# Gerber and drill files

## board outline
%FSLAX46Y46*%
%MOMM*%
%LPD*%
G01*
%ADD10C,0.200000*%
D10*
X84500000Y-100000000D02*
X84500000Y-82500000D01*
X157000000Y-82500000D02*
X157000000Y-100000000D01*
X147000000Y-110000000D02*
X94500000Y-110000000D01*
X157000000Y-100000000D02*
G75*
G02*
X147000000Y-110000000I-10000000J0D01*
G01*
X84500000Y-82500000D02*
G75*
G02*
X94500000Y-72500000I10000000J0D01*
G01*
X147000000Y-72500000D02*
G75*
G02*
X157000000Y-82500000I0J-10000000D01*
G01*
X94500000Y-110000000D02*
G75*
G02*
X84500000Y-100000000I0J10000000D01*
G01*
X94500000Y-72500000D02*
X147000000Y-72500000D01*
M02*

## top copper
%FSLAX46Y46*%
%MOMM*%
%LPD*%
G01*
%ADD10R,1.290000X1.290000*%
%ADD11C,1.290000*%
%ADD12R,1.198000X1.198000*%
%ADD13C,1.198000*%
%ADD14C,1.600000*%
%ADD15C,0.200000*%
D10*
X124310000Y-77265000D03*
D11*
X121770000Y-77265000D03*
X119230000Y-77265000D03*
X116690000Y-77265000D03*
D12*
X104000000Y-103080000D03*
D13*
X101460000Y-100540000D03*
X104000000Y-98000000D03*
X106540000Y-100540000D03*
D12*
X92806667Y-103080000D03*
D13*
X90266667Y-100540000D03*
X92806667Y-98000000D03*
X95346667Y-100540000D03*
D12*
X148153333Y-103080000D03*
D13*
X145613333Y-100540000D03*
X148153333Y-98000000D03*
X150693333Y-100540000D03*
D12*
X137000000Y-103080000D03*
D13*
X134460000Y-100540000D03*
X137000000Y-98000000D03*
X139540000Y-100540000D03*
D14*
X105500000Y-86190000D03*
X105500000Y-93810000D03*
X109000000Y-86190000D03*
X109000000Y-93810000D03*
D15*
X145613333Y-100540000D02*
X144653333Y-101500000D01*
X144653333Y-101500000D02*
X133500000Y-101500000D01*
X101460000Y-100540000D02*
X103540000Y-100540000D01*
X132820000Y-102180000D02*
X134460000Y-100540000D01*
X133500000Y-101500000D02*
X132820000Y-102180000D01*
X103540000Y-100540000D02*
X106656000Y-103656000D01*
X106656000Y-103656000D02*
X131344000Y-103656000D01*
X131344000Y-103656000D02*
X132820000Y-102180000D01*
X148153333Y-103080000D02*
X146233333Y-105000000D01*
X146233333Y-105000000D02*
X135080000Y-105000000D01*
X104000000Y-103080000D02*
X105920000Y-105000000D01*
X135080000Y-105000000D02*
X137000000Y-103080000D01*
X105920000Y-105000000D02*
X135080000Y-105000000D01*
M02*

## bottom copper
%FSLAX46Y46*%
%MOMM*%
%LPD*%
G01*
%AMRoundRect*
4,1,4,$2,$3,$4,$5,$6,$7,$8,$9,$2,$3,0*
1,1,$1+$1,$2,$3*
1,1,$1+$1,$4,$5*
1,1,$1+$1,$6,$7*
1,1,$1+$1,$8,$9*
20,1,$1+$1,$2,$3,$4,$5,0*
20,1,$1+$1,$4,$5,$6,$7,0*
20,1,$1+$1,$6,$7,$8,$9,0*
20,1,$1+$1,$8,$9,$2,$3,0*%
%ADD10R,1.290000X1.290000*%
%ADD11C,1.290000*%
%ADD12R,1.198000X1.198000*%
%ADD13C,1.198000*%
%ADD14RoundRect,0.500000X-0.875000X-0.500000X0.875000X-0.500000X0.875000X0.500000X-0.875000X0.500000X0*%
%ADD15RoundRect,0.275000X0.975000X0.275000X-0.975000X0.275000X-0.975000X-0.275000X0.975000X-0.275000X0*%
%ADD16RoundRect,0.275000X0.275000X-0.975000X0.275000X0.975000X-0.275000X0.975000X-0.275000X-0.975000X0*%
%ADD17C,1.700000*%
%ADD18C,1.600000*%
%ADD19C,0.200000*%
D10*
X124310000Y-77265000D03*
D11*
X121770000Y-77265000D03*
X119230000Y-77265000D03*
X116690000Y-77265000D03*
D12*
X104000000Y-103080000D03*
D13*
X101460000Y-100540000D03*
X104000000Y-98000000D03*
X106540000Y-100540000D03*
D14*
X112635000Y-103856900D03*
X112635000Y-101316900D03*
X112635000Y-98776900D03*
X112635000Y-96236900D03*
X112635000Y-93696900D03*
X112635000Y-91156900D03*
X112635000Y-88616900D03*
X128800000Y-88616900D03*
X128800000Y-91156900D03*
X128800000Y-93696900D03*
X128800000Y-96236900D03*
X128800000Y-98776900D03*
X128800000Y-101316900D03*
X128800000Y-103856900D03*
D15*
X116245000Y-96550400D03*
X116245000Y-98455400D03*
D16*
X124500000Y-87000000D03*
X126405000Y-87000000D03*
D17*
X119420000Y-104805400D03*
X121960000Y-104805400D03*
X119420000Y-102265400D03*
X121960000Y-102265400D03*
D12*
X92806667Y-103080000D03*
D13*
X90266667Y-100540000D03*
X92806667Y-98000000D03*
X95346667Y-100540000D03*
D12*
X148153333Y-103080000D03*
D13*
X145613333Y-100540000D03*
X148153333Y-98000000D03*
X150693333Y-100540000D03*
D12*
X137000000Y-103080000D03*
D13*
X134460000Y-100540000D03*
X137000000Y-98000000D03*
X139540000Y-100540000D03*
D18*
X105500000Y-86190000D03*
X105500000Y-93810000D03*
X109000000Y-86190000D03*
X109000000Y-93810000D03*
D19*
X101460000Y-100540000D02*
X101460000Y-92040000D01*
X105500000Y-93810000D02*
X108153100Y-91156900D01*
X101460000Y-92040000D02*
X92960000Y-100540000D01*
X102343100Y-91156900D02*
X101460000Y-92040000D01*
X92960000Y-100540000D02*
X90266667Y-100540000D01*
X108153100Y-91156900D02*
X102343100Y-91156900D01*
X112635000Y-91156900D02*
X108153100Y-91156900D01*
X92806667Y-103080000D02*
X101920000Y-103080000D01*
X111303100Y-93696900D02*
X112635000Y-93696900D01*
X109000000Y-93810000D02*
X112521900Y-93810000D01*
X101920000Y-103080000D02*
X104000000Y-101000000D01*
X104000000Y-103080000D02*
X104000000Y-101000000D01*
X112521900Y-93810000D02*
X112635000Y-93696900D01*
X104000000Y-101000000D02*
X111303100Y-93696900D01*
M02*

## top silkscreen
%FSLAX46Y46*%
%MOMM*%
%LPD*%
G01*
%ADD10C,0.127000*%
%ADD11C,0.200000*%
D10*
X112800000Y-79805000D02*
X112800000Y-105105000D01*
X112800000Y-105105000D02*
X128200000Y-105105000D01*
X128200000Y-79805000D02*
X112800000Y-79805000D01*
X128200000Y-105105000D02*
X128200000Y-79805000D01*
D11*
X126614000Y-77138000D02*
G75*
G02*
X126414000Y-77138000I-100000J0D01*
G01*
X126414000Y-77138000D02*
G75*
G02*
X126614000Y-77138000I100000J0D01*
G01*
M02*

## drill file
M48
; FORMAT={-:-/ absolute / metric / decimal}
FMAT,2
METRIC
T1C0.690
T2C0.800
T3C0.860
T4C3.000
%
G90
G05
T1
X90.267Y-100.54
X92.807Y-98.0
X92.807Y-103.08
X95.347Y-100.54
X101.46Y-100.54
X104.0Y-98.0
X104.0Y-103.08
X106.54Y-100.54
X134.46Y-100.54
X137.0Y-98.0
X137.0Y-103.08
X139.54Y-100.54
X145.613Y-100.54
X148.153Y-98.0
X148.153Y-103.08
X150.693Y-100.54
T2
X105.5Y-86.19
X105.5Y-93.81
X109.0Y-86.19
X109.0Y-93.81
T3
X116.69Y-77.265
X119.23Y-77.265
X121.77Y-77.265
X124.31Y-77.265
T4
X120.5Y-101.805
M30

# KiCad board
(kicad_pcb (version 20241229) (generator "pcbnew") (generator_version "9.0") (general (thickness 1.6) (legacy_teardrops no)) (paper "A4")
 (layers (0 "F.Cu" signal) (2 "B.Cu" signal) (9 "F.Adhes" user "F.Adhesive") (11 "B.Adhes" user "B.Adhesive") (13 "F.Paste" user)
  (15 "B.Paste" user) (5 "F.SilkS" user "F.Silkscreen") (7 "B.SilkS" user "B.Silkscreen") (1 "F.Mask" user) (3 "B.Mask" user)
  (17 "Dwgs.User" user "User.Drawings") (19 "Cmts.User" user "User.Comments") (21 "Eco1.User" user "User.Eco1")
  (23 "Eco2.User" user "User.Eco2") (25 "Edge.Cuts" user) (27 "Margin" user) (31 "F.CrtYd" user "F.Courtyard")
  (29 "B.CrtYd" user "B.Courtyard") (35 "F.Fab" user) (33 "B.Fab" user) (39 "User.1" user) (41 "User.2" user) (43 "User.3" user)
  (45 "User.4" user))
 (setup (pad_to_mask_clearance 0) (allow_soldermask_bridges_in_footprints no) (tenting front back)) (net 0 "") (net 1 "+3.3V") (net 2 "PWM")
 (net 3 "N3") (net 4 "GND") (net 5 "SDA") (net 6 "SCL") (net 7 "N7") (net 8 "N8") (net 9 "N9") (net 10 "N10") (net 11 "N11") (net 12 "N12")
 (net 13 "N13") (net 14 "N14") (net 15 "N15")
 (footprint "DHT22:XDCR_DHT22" (layer "F.Cu") (at 120.5 92.455 180)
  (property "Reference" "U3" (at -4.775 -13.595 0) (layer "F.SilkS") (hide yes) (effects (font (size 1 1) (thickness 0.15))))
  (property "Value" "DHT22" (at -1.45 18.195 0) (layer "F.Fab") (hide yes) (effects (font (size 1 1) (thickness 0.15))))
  (fp_line (start 7.7 12.65) (end 7.7 -12.65) (stroke (width 0.127) (type solid)) (layer "F.SilkS"))
  (fp_line (start 7.7 -12.65) (end -7.7 -12.65) (stroke (width 0.127) (type solid)) (layer "F.SilkS"))
  (fp_line (start -7.7 12.65) (end 7.7 12.65) (stroke (width 0.127) (type solid)) (layer "F.SilkS"))
  (fp_line (start -7.7 -12.65) (end -7.7 12.65) (stroke (width 0.127) (type solid)) (layer "F.SilkS"))
  (fp_circle (center -6.014 15.317) (end -5.914 15.317) (stroke (width 0.2) (type solid)) (fill no) (layer "F.SilkS"))
  (pad "" np_thru_hole circle (at 0 -9.35 180) (size 3 3) (drill 3) (layers "*.Cu" "*.Mask"))
  (pad "1" thru_hole rect (at -3.81 15.19 180) (size 1.29 1.29) (drill 0.86) (layers "*.Cu" "*.Mask") (remove_unused_layers no)
   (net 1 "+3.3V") (solder_mask_margin 0.102))
  (pad "2" thru_hole circle (at -1.27 15.19 180) (size 1.29 1.29) (drill 0.86) (layers "*.Cu" "*.Mask") (remove_unused_layers no)
   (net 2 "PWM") (solder_mask_margin 0.102))
  (pad "3" thru_hole circle (at 1.27 15.19 180) (size 1.29 1.29) (drill 0.86) (layers "*.Cu" "*.Mask") (remove_unused_layers no)
   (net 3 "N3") (solder_mask_margin 0.102))
  (pad "4" thru_hole circle (at 3.81 15.19 180) (size 1.29 1.29) (drill 0.86) (layers "*.Cu" "*.Mask") (remove_unused_layers no)
   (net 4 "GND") (solder_mask_margin 0.102)))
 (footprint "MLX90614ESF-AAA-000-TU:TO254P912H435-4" (layer "B.Cu") (at 104 100.54 90)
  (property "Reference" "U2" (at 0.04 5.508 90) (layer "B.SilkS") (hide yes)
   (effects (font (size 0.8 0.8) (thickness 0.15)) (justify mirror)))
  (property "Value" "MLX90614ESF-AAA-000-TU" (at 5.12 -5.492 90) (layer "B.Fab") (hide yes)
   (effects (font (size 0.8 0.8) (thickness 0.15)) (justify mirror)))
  (pad "1" thru_hole rect (at -2.54 0 90) (size 1.198 1.198) (drill 0.69) (layers "*.Cu" "*.Mask") (remove_unused_layers no) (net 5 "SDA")
   (solder_mask_margin 0.102))
  (pad "2" thru_hole circle (at 0 -2.54 90) (size 1.198 1.198) (drill 0.69) (layers "*.Cu" "*.Mask") (remove_unused_layers no) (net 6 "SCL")
   (solder_mask_margin 0.102))
  (pad "3" thru_hole circle (at 2.54 0 90) (size 1.198 1.198) (drill 0.69) (layers "*.Cu" "*.Mask") (remove_unused_layers no)
   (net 1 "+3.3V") (solder_mask_margin 0.102))
  (pad "4" thru_hole circle (at 0 2.54 90) (size 1.198 1.198) (drill 0.69) (layers "*.Cu" "*.Mask") (remove_unused_layers no) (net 4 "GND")
   (solder_mask_margin 0.102)))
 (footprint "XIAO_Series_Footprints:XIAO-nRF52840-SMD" (layer "B.Cu") (at 111.8 85.7369)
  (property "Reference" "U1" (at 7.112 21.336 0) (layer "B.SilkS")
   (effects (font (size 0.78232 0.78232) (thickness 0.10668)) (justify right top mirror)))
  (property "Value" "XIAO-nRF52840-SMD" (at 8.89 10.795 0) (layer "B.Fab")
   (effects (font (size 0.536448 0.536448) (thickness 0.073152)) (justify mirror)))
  (pad "1" smd roundrect (at 0.835 18.12) (size 2.75 2) (layers "B.Cu" "B.Mask" "B.Paste") (roundrect_rratio 0.25) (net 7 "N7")
   (solder_mask_margin 0.0508) (thermal_bridge_angle 45))
  (pad "2" smd roundrect (at 0.835 15.58) (size 2.75 2) (layers "B.Cu" "B.Mask" "B.Paste") (roundrect_rratio 0.25) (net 2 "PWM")
   (solder_mask_margin 0.0508) (thermal_bridge_angle 45))
  (pad "3" smd roundrect (at 0.835 13.04) (size 2.75 2) (layers "B.Cu" "B.Mask" "B.Paste") (roundrect_rratio 0.25) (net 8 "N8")
   (solder_mask_margin 0.0508) (thermal_bridge_angle 45))
  (pad "4" smd roundrect (at 0.835 10.5) (size 2.75 2) (layers "B.Cu" "B.Mask" "B.Paste") (roundrect_rratio 0.25) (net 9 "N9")
   (solder_mask_margin 0.0508) (thermal_bridge_angle 45))
  (pad "5" smd roundrect (at 0.835 7.96) (size 2.75 2) (layers "B.Cu" "B.Mask" "B.Paste") (roundrect_rratio 0.25) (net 5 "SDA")
   (solder_mask_margin 0.0508) (thermal_bridge_angle 45))
  (pad "6" smd roundrect (at 0.835 5.42) (size 2.75 2) (layers "B.Cu" "B.Mask" "B.Paste") (roundrect_rratio 0.25) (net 6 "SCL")
   (solder_mask_margin 0.0508) (thermal_bridge_angle 45))
  (pad "7" smd roundrect (at 0.835 2.88) (size 2.75 2) (layers "B.Cu" "B.Mask" "B.Paste") (roundrect_rratio 0.25) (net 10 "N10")
   (solder_mask_margin 0.0508) (thermal_bridge_angle 45))
  (pad "8" smd roundrect (at 17 2.88) (size 2.75 2) (layers "B.Cu" "B.Mask" "B.Paste") (roundrect_rratio 0.25) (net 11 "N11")
   (solder_mask_margin 0.0508) (thermal_bridge_angle 45))
  (pad "9" smd roundrect (at 17 5.42) (size 2.75 2) (layers "B.Cu" "B.Mask" "B.Paste") (roundrect_rratio 0.25) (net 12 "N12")
   (solder_mask_margin 0.0508) (thermal_bridge_angle 45))
  (pad "10" smd roundrect (at 17 7.96) (size 2.75 2) (layers "B.Cu" "B.Mask" "B.Paste") (roundrect_rratio 0.25) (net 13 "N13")
   (solder_mask_margin 0.0508) (thermal_bridge_angle 45))
  (pad "11" smd roundrect (at 17 10.5) (size 2.75 2) (layers "B.Cu" "B.Mask" "B.Paste") (roundrect_rratio 0.25) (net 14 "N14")
   (solder_mask_margin 0.0508) (thermal_bridge_angle 45))
  (pad "12" smd roundrect (at 17 13.04) (size 2.75 2) (layers "B.Cu" "B.Mask" "B.Paste") (roundrect_rratio 0.25) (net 1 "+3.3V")
   (solder_mask_margin 0.0508) (thermal_bridge_angle 45))
  (pad "13" smd roundrect (at 17 15.58) (size 2.75 2) (layers "B.Cu" "B.Mask" "B.Paste") (roundrect_rratio 0.25) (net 4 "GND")
   (solder_mask_margin 0.0508) (thermal_bridge_angle 45))
  (pad "14" smd roundrect (at 17 18.12) (size 2.75 2) (layers "B.Cu" "B.Mask" "B.Paste") (roundrect_rratio 0.25) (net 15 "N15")
   (solder_mask_margin 0.0508) (thermal_bridge_angle 45))
  (pad "15" smd roundrect (at 4.445 10.8135 180) (size 2.5 1.1) (layers "B.Cu" "B.Mask" "B.Paste") (roundrect_rratio 0.25)
   (solder_mask_margin 0.0508) (thermal_bridge_angle 45))
  (pad "16" smd roundrect (at 4.445 12.7185 180) (size 2.5 1.1) (layers "B.Cu" "B.Mask" "B.Paste") (roundrect_rratio 0.25)
   (solder_mask_margin 0.0508) (thermal_bridge_angle 45))
  (pad "17" smd roundrect (at 12.7 1.2631 90) (size 2.5 1.1) (layers "B.Cu" "B.Mask" "B.Paste") (roundrect_rratio 0.25)
   (solder_mask_margin 0.0508) (thermal_bridge_angle 45))
  (pad "18" smd roundrect (at 14.605 1.2631 90) (size 2.5 1.1) (layers "B.Cu" "B.Mask" "B.Paste") (roundrect_rratio 0.25)
   (solder_mask_margin 0.0508) (thermal_bridge_angle 45))
  (pad "19" smd circle (at 7.62 19.0685) (size 1.7 1.7) (layers "B.Cu" "B.Mask" "B.Paste"))
  (pad "20" smd circle (at 10.16 19.0685) (size 1.7 1.7) (layers "B.Cu" "B.Mask" "B.Paste"))
  (pad "21" smd circle (at 7.62 16.5285) (size 1.7 1.7) (layers "B.Cu" "B.Mask" "B.Paste"))
  (pad "22" smd circle (at 10.16 16.5285) (size 1.7 1.7) (layers "B.Cu" "B.Mask" "B.Paste")))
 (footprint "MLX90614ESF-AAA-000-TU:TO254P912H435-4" (layer "B.Cu") (at 92.806667 100.54 90)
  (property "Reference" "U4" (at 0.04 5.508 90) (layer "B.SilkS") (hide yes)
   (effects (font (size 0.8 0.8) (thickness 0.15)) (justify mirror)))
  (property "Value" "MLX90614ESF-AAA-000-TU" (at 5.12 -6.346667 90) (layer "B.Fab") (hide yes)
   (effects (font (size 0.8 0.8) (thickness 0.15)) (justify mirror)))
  (pad "1" thru_hole rect (at -2.54 0 90) (size 1.198 1.198) (drill 0.69) (layers "*.Cu" "*.Mask") (remove_unused_layers no) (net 5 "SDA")
   (solder_mask_margin 0.102))
  (pad "2" thru_hole circle (at 0 -2.54 90) (size 1.198 1.198) (drill 0.69) (layers "*.Cu" "*.Mask") (remove_unused_layers no) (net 6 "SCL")
   (solder_mask_margin 0.102))
  (pad "3" thru_hole circle (at 2.54 0 90) (size 1.198 1.198) (drill 0.69) (layers "*.Cu" "*.Mask") (remove_unused_layers no)
   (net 1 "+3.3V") (solder_mask_margin 0.102))
  (pad "4" thru_hole circle (at 0 2.54 90) (size 1.198 1.198) (drill 0.69) (layers "*.Cu" "*.Mask") (remove_unused_layers no) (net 4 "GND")
   (solder_mask_margin 0.102)))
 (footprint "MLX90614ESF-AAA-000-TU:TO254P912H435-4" (layer "B.Cu") (at 148.153333 100.54 90)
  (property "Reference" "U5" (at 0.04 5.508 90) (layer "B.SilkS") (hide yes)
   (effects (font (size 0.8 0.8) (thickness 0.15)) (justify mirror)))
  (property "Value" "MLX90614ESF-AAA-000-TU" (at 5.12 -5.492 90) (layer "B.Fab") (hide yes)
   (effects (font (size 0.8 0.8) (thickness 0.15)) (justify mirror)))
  (pad "1" thru_hole rect (at -2.54 0 90) (size 1.198 1.198) (drill 0.69) (layers "*.Cu" "*.Mask") (remove_unused_layers no) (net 5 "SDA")
   (solder_mask_margin 0.102))
  (pad "2" thru_hole circle (at 0 -2.54 90) (size 1.198 1.198) (drill 0.69) (layers "*.Cu" "*.Mask") (remove_unused_layers no) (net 6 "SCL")
   (solder_mask_margin 0.102))
  (pad "3" thru_hole circle (at 2.54 0 90) (size 1.198 1.198) (drill 0.69) (layers "*.Cu" "*.Mask") (remove_unused_layers no)
   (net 1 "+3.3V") (solder_mask_margin 0.102))
  (pad "4" thru_hole circle (at 0 2.54 90) (size 1.198 1.198) (drill 0.69) (layers "*.Cu" "*.Mask") (remove_unused_layers no) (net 4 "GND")
   (solder_mask_margin 0.102)))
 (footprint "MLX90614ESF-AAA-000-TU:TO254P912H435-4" (layer "B.Cu") (at 137 100.54 90)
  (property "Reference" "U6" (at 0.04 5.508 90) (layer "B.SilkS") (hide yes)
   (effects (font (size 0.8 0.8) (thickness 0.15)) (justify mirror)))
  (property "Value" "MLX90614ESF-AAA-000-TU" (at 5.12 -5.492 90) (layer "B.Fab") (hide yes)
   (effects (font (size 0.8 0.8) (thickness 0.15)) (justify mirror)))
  (pad "1" thru_hole rect (at -2.54 0 90) (size 1.198 1.198) (drill 0.69) (layers "*.Cu" "*.Mask") (remove_unused_layers no) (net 5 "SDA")
   (solder_mask_margin 0.102))
  (pad "2" thru_hole circle (at 0 -2.54 90) (size 1.198 1.198) (drill 0.69) (layers "*.Cu" "*.Mask") (remove_unused_layers no) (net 6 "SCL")
   (solder_mask_margin 0.102))
  (pad "3" thru_hole circle (at 2.54 0 90) (size 1.198 1.198) (drill 0.69) (layers "*.Cu" "*.Mask") (remove_unused_layers no)
   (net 1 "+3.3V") (solder_mask_margin 0.102))
  (pad "4" thru_hole circle (at 0 2.54 90) (size 1.198 1.198) (drill 0.69) (layers "*.Cu" "*.Mask") (remove_unused_layers no) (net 4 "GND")
   (solder_mask_margin 0.102)))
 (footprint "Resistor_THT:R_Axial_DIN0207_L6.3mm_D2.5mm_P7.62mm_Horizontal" (layer "B.Cu") (at 105.5 86.19 -90)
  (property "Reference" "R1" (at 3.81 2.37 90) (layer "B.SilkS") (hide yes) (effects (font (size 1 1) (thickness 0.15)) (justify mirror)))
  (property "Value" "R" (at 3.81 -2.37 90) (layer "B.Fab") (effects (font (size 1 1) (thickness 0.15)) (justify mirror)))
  (pad "1" thru_hole circle (at 0 0 270) (size 1.6 1.6) (drill 0.8) (layers "*.Cu" "*.Mask") (remove_unused_layers no) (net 1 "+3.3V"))
  (pad "2" thru_hole circle (at 7.62 0 270) (size 1.6 1.6) (drill 0.8) (layers "*.Cu" "*.Mask") (remove_unused_layers no) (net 6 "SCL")))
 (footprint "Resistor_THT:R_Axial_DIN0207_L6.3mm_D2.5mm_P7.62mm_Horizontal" (layer "B.Cu") (at 109 86.19 -90)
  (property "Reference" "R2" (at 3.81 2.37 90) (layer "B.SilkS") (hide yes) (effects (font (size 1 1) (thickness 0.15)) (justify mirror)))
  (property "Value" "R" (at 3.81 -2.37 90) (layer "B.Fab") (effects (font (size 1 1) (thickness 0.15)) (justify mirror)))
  (pad "1" thru_hole circle (at 0 0 270) (size 1.6 1.6) (drill 0.8) (layers "*.Cu" "*.Mask") (remove_unused_layers no) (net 1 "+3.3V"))
  (pad "2" thru_hole circle (at 7.62 0 270) (size 1.6 1.6) (drill 0.8) (layers "*.Cu" "*.Mask") (remove_unused_layers no) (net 5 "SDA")))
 (gr_line (start 84.5 100) (end 84.5 82.5) (stroke (width 0.2) (type default)) (layer "Edge.Cuts"))
 (gr_line (start 157 82.5) (end 157 100) (stroke (width 0.2) (type default)) (layer "Edge.Cuts"))
 (gr_line (start 147 110) (end 94.5 110) (stroke (width 0.2) (type default)) (layer "Edge.Cuts"))
 (gr_arc (start 157 100) (mid 154.071068 107.071068) (end 147 110) (stroke (width 0.2) (type default)) (layer "Edge.Cuts"))
 (gr_arc (start 84.5 82.5) (mid 87.428932 75.428932) (end 94.5 72.5) (stroke (width 0.2) (type default)) (layer "Edge.Cuts"))
 (gr_arc (start 147 72.5) (mid 154.071068 75.428932) (end 157 82.5) (stroke (width 0.2) (type default)) (layer "Edge.Cuts"))
 (gr_arc (start 94.5 110) (mid 87.428932 107.071068) (end 84.5 100) (stroke (width 0.2) (type default)) (layer "Edge.Cuts"))
 (gr_line (start 94.5 72.5) (end 147 72.5) (stroke (width 0.2) (type default)) (layer "Edge.Cuts"))
 (segment (start 145.613333 100.54) (end 144.653333 101.5) (width 0.2) (layer "F.Cu") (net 6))
 (segment (start 144.653333 101.5) (end 133.5 101.5) (width 0.2) (layer "F.Cu") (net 6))
 (segment (start 101.46 100.54) (end 103.54 100.54) (width 0.2) (layer "F.Cu") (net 6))
 (segment (start 132.82 102.18) (end 134.46 100.54) (width 0.2) (layer "F.Cu") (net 6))
 (segment (start 133.5 101.5) (end 132.82 102.18) (width 0.2) (layer "F.Cu") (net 6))
 (segment (start 103.54 100.54) (end 106.656 103.656) (width 0.2) (layer "F.Cu") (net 6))
 (segment (start 106.656 103.656) (end 131.344 103.656) (width 0.2) (layer "F.Cu") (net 6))
 (segment (start 131.344 103.656) (end 132.82 102.18) (width 0.2) (layer "F.Cu") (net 6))
 (segment (start 101.46 100.54) (end 101.46 92.04) (width 0.2) (layer "B.Cu") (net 6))
 (segment (start 105.5 93.81) (end 108.1531 91.1569) (width 0.2) (layer "B.Cu") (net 6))
 (segment (start 101.46 92.04) (end 92.96 100.54) (width 0.2) (layer "B.Cu") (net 6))
 (segment (start 102.3431 91.1569) (end 101.46 92.04) (width 0.2) (layer "B.Cu") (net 6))
 (segment (start 92.96 100.54) (end 90.266667 100.54) (width 0.2) (layer "B.Cu") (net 6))
 (segment (start 108.1531 91.1569) (end 102.3431 91.1569) (width 0.2) (layer "B.Cu") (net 6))
 (segment (start 112.635 91.1569) (end 108.1531 91.1569) (width 0.2) (layer "B.Cu") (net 6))
 (segment (start 148.153333 103.08) (end 146.233333 105) (width 0.2) (layer "F.Cu") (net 5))
 (segment (start 146.233333 105) (end 135.08 105) (width 0.2) (layer "F.Cu") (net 5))
 (segment (start 104 103.08) (end 105.92 105) (width 0.2) (layer "F.Cu") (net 5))
 (segment (start 135.08 105) (end 137 103.08) (width 0.2) (layer "F.Cu") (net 5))
 (segment (start 105.92 105) (end 135.08 105) (width 0.2) (layer "F.Cu") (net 5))
 (segment (start 92.806667 103.08) (end 101.92 103.08) (width 0.2) (layer "B.Cu") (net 5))
 (segment (start 111.3031 93.6969) (end 112.635 93.6969) (width 0.2) (layer "B.Cu") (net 5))
 (segment (start 109 93.81) (end 112.5219 93.81) (width 0.2) (layer "B.Cu") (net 5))
 (segment (start 101.92 103.08) (end 104 101) (width 0.2) (layer "B.Cu") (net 5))
 (segment (start 104 103.08) (end 104 101) (width 0.2) (layer "B.Cu") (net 5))
 (segment (start 112.5219 93.81) (end 112.635 93.6969) (width 0.2) (layer "B.Cu") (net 5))
 (segment (start 104 101) (end 111.3031 93.6969) (width 0.2) (layer "B.Cu") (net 5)))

